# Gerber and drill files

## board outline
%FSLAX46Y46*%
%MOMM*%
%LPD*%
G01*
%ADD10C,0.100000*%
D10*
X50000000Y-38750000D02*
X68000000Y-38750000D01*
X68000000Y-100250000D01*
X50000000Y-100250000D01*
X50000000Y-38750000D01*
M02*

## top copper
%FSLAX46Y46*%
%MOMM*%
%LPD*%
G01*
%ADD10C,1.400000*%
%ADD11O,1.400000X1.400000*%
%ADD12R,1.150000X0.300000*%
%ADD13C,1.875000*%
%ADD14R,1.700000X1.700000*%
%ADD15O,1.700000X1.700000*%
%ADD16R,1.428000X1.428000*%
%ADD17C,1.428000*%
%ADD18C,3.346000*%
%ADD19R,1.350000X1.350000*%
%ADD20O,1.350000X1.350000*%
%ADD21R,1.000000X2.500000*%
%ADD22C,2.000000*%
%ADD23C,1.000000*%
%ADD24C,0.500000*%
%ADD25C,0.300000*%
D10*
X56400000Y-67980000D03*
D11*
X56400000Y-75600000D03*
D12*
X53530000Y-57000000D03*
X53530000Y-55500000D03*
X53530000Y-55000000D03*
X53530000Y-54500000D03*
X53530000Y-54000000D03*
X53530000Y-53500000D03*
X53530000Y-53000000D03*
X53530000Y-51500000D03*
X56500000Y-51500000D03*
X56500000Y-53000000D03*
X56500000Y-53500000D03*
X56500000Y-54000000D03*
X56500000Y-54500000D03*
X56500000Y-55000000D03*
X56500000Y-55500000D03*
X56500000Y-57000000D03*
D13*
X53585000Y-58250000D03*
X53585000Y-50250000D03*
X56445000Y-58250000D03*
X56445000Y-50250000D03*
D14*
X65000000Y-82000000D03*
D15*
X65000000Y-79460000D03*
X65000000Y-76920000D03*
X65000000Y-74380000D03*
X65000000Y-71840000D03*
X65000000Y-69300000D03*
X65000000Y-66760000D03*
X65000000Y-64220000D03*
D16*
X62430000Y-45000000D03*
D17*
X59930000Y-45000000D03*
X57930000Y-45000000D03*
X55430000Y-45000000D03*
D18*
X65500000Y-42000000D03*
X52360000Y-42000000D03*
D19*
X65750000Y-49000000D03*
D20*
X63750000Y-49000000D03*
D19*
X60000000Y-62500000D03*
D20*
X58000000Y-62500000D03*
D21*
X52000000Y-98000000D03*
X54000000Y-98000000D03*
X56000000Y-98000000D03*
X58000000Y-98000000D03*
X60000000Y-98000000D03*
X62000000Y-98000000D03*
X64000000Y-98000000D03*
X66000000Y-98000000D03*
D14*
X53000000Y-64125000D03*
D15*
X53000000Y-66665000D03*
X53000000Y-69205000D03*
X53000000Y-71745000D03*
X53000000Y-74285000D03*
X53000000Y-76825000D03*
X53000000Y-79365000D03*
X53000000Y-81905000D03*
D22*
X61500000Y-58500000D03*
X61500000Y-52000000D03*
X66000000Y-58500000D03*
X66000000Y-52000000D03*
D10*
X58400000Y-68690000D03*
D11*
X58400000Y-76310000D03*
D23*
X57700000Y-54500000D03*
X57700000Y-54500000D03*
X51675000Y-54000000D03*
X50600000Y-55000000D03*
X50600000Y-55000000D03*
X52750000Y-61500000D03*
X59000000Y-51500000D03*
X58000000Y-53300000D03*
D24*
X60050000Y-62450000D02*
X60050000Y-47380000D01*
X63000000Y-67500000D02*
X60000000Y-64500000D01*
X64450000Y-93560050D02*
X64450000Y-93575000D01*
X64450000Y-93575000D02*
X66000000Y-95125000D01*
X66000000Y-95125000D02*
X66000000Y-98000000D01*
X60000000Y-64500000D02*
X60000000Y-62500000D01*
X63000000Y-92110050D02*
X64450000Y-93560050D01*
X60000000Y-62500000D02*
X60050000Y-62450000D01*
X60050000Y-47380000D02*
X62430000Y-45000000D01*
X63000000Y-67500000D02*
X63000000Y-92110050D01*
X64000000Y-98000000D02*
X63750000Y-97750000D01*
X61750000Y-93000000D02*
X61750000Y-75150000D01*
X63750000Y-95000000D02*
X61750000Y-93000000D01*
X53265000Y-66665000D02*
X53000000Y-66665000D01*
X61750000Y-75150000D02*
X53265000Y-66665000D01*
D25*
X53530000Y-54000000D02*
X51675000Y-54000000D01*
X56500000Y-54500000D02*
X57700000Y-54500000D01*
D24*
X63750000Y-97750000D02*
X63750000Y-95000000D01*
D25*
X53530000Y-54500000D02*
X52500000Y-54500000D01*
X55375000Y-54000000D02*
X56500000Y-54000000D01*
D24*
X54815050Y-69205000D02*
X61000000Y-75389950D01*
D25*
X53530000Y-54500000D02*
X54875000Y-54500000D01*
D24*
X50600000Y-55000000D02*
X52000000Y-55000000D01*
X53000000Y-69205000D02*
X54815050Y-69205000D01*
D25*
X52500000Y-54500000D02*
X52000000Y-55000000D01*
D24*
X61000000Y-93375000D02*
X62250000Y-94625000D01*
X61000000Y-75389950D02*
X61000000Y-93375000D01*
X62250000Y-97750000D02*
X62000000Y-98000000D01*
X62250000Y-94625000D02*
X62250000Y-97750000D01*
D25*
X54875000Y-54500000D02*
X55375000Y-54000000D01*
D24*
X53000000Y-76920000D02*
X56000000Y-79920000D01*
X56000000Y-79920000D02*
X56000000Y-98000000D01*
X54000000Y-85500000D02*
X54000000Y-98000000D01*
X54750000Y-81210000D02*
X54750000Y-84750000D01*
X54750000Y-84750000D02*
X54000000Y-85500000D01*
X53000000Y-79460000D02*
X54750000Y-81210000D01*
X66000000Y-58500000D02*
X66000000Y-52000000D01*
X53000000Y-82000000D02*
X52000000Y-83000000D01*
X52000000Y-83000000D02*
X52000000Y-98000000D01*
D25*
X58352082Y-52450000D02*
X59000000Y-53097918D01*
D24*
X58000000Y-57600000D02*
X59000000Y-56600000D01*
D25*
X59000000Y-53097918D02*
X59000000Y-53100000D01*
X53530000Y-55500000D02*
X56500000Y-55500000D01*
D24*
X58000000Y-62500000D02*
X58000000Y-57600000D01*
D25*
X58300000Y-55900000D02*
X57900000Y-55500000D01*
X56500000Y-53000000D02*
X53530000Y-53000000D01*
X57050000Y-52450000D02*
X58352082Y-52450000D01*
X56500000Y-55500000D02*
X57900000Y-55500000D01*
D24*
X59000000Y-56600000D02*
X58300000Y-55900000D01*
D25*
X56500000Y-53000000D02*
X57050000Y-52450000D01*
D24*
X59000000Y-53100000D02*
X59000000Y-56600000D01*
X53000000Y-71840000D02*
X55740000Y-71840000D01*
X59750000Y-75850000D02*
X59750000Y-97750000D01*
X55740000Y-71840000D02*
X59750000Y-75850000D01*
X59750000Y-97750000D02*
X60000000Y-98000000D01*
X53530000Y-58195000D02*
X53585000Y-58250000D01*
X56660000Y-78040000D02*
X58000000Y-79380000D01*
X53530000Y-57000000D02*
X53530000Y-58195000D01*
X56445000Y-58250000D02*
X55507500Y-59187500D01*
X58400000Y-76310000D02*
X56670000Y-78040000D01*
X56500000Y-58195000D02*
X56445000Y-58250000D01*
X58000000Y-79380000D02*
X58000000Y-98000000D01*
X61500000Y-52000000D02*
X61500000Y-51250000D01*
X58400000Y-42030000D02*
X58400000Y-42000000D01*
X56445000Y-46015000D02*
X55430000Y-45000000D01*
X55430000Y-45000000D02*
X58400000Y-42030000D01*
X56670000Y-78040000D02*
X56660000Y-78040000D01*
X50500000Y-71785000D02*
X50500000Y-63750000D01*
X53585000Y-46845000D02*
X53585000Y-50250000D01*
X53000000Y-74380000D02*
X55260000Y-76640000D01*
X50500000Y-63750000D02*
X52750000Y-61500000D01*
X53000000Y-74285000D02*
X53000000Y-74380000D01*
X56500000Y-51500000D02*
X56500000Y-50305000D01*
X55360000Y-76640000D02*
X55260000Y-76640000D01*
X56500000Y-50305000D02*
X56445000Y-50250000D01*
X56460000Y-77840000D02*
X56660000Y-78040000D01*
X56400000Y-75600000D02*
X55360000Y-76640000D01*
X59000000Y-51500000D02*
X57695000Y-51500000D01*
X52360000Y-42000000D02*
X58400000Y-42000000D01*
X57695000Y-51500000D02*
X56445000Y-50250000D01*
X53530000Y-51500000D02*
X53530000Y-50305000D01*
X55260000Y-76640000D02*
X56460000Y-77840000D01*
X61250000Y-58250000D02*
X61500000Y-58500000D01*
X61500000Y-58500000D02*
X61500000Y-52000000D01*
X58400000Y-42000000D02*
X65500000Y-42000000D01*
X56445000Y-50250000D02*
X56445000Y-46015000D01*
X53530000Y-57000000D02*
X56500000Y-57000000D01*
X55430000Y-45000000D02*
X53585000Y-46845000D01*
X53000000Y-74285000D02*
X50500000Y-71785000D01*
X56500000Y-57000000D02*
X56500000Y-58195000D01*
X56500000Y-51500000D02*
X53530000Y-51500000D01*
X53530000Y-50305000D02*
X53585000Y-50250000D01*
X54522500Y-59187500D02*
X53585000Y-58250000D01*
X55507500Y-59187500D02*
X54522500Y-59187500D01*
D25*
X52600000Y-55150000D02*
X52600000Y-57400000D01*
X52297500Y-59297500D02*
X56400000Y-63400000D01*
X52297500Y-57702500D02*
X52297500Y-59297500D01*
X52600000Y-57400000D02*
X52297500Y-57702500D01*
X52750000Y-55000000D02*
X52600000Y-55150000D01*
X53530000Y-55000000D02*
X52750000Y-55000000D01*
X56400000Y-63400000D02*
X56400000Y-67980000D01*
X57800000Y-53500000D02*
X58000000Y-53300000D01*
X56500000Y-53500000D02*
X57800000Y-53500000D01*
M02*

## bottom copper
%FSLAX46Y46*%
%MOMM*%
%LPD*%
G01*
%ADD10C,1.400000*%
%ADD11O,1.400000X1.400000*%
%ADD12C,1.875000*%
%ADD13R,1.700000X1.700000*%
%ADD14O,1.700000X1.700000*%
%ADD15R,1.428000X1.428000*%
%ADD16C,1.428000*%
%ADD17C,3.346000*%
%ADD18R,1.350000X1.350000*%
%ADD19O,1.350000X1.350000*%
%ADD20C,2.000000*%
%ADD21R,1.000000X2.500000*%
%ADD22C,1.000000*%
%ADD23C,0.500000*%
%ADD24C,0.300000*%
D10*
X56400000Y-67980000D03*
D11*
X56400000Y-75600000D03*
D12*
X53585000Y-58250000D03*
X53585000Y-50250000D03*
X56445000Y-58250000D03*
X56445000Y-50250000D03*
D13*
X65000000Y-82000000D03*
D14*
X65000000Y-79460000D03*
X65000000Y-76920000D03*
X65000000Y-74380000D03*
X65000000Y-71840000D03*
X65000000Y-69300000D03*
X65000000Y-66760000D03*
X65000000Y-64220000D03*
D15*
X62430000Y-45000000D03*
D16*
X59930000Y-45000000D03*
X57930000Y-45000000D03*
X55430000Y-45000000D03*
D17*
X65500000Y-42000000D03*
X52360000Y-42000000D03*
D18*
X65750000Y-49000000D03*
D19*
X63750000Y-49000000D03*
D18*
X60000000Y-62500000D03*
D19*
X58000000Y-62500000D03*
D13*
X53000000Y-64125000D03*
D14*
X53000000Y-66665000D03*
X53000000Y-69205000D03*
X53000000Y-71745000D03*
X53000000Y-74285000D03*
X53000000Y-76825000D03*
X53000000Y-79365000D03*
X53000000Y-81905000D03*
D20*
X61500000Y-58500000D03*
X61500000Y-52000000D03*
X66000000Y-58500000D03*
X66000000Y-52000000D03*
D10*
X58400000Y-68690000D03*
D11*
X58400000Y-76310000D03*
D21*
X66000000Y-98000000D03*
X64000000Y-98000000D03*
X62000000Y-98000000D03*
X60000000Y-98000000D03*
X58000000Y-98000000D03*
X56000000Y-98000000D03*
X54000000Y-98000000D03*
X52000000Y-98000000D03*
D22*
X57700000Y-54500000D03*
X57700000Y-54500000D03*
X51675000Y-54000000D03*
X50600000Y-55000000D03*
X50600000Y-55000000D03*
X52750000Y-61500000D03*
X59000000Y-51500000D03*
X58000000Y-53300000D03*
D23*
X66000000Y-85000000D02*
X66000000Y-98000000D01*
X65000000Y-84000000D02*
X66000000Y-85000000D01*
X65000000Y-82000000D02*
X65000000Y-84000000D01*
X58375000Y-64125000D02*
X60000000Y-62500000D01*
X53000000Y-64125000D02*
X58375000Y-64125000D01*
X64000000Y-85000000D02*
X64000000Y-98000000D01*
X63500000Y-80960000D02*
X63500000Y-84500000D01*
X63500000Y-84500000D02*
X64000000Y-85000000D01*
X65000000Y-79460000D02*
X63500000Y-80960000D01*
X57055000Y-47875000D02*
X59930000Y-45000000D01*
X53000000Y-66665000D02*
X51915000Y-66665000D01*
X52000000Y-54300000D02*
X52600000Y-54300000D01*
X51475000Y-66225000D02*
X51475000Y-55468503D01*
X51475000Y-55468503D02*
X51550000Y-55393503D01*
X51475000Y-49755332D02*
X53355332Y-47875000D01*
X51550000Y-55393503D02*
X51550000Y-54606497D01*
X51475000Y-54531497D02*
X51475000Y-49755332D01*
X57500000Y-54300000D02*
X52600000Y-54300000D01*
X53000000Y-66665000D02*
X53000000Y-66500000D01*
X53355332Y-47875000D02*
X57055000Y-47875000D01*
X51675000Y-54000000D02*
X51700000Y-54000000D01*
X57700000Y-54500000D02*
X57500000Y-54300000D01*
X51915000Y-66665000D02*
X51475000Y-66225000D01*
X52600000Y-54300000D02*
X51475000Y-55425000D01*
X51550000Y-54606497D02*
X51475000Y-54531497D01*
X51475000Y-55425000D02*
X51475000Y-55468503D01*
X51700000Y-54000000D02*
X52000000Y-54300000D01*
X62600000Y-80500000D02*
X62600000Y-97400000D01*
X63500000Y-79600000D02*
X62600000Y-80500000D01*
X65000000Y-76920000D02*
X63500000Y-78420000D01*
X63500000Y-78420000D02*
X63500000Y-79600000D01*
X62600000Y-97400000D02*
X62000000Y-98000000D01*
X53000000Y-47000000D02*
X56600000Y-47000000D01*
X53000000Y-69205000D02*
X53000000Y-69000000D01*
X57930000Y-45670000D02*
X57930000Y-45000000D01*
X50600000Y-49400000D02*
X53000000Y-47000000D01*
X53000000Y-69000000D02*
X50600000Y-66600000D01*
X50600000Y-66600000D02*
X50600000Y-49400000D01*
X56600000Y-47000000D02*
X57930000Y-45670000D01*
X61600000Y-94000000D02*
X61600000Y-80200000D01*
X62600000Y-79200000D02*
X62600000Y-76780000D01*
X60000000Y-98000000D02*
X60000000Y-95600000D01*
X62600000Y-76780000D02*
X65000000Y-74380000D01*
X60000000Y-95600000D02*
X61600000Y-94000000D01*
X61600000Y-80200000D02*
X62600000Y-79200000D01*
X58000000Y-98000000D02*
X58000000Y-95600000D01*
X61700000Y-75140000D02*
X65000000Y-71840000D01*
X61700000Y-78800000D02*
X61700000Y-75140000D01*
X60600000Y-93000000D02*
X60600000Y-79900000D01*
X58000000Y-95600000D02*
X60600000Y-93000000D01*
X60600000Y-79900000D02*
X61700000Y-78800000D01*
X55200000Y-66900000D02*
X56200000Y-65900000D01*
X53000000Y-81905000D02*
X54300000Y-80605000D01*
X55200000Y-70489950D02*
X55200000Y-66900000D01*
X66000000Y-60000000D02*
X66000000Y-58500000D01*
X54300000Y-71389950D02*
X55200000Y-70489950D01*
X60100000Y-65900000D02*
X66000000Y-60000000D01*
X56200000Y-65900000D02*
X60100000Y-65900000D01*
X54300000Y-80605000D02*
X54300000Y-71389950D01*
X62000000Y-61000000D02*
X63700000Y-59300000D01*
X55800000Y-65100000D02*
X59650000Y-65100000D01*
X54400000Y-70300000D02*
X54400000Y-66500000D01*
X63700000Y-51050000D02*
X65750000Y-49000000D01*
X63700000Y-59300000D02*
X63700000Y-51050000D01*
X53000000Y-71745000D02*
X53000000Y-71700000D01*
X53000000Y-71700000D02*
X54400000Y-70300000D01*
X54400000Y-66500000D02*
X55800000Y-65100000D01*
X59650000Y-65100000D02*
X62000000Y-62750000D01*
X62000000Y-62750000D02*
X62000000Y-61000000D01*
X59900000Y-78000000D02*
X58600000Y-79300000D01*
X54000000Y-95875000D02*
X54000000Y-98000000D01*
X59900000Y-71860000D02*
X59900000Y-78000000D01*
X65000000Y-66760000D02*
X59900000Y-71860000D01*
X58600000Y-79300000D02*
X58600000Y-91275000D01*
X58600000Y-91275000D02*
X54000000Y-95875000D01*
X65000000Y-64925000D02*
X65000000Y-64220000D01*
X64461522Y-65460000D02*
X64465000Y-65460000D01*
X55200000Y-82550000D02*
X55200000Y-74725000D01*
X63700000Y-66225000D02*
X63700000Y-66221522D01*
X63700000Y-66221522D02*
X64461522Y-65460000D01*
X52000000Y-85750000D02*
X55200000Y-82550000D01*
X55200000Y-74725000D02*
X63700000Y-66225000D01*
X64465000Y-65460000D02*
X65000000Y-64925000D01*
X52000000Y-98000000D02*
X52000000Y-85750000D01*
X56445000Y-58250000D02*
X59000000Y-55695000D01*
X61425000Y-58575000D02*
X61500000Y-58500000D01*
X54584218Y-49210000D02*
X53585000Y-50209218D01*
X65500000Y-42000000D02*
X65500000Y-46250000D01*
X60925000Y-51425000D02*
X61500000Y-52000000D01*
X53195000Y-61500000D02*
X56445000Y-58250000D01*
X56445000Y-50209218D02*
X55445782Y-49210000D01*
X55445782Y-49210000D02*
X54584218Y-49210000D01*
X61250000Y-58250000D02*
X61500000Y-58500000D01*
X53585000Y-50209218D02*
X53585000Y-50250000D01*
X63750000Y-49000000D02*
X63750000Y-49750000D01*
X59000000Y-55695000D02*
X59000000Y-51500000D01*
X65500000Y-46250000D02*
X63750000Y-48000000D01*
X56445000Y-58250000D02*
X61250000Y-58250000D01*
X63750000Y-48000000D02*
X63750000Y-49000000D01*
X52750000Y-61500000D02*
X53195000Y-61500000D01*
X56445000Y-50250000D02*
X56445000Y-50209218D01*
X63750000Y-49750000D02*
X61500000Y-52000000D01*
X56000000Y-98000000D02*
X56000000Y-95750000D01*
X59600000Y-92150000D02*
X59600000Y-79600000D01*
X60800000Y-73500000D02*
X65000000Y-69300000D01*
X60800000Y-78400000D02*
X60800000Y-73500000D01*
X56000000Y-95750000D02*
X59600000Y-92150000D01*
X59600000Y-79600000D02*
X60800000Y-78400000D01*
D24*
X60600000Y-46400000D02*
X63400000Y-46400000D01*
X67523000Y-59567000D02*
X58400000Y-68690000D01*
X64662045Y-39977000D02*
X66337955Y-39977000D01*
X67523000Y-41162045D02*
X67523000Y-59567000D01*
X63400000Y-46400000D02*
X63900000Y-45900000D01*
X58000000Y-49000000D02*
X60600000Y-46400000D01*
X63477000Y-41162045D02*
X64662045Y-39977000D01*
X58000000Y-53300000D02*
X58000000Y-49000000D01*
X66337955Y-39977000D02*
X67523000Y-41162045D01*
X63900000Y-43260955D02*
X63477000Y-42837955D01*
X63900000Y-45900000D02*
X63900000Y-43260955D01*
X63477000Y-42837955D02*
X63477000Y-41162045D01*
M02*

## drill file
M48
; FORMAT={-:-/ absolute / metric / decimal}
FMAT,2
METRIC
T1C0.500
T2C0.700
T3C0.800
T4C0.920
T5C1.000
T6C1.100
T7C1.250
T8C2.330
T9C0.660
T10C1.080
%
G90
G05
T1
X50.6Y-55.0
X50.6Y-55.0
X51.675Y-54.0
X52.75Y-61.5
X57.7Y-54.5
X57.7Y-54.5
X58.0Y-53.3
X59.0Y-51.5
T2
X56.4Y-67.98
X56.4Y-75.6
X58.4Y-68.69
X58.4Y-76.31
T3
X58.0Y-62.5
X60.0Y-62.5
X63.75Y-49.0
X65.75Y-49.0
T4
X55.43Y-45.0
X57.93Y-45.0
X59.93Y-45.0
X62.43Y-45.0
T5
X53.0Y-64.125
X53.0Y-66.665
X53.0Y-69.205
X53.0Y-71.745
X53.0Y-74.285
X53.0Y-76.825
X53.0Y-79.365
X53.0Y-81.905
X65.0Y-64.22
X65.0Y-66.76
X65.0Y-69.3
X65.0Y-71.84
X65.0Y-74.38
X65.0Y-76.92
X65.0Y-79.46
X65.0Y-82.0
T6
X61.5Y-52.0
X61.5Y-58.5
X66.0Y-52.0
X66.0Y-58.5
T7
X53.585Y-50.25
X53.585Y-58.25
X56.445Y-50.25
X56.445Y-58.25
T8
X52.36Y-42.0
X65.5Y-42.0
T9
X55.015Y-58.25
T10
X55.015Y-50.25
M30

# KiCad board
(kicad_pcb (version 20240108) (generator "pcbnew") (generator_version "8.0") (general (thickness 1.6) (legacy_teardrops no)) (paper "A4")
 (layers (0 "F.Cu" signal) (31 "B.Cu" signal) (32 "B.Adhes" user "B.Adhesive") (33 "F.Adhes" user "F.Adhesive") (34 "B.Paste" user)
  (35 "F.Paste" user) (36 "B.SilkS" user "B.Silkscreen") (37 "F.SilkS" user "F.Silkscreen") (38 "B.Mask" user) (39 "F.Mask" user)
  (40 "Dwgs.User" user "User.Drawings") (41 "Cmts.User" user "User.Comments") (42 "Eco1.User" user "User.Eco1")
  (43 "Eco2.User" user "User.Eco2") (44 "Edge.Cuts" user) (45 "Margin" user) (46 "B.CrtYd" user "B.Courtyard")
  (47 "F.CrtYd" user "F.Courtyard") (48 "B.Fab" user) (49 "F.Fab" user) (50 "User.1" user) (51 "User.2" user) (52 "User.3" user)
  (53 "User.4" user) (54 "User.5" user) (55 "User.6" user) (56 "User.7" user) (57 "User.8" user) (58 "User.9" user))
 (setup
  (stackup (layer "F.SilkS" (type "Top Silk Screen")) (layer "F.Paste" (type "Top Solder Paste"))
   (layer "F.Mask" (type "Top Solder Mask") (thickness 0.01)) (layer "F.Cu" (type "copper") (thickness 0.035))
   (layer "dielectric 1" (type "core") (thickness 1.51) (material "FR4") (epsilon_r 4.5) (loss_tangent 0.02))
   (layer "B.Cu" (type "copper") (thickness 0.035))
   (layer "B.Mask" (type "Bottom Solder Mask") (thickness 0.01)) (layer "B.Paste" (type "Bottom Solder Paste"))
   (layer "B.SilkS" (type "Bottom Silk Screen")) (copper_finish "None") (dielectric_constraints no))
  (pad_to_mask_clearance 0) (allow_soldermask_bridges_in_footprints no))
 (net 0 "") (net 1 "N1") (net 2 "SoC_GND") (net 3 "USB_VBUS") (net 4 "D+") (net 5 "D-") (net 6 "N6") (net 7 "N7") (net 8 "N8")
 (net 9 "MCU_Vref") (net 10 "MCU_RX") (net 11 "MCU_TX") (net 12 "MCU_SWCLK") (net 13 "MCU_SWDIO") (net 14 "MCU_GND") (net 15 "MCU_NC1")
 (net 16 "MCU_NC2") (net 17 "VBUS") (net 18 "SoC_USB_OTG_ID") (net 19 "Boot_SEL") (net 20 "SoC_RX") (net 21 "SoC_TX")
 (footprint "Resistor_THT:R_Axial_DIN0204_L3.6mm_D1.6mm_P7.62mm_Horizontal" (layer "F.Cu") (at 56.4 67.98 -90)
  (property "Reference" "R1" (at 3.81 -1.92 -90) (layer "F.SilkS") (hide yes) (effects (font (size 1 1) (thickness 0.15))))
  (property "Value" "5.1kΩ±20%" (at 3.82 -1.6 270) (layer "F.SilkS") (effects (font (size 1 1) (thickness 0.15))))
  (pad "1" thru_hole circle (at 0 0 270) (size 1.4 1.4) (drill 0.7) (layers "*.Cu" "*.Mask") (remove_unused_layers no) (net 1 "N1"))
  (pad "2" thru_hole oval (at 7.62 0 270) (size 1.4 1.4) (drill 0.7) (layers "*.Cu" "*.Mask") (remove_unused_layers no) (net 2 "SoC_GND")))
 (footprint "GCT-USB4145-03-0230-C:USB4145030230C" (layer "F.Cu") (at 55.015 54.25 90)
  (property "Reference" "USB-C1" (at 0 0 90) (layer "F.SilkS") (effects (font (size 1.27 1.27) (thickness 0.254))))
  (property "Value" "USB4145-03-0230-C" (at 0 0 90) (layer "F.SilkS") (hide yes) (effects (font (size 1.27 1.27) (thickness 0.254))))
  (pad "" np_thru_hole circle (at -4 0 90) (size 0.66 0.66) (drill 0.66) (layers "*.Cu" "*.Mask"))
  (pad "" np_thru_hole circle (at 4 0 90) (size 1.08 1.08) (drill 1.08) (layers "*.Cu" "*.Mask"))
  (pad "A1" smd rect (at -2.75 -1.485 90) (size 0.3 1.15) (layers "F.Cu" "F.Mask") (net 2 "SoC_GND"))
  (pad "A4" smd rect (at -1.25 -1.485 90) (size 0.3 1.15) (layers "F.Cu" "F.Mask") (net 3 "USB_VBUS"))
  (pad "A5" smd rect (at -0.75 -1.485 90) (size 0.3 1.15) (layers "F.Cu" "F.Mask") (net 1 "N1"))
  (pad "A6" smd rect (at -0.25 -1.485 90) (size 0.3 1.15) (layers "F.Cu" "F.Mask") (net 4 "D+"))
  (pad "A7" smd rect (at 0.25 -1.485 90) (size 0.3 1.15) (layers "F.Cu" "F.Mask") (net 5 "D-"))
  (pad "A8" smd rect (at 0.75 -1.485 90) (size 0.3 1.15) (layers "F.Cu" "F.Mask") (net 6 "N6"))
  (pad "A9" smd rect (at 1.25 -1.485 90) (size 0.3 1.15) (layers "F.Cu" "F.Mask") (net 3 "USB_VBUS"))
  (pad "A12" smd rect (at 2.75 -1.485 90) (size 0.3 1.15) (layers "F.Cu" "F.Mask") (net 2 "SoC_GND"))
  (pad "B1" smd rect (at 2.75 1.485 90) (size 0.3 1.15) (layers "F.Cu" "F.Mask") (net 2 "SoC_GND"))
  (pad "B4" smd rect (at 1.25 1.485 90) (size 0.3 1.15) (layers "F.Cu" "F.Mask") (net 3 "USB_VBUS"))
  (pad "B5" smd rect (at 0.75 1.485 90) (size 0.3 1.15) (layers "F.Cu" "F.Mask") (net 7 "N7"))
  (pad "B6" smd rect (at 0.25 1.485 90) (size 0.3 1.15) (layers "F.Cu" "F.Mask") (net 4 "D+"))
  (pad "B7" smd rect (at -0.25 1.485 90) (size 0.3 1.15) (layers "F.Cu" "F.Mask") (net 5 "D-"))
  (pad "B8" smd rect (at -0.75 1.485 90) (size 0.3 1.15) (layers "F.Cu" "F.Mask") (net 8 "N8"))
  (pad "B9" smd rect (at -1.25 1.485 90) (size 0.3 1.15) (layers "F.Cu" "F.Mask") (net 3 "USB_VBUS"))
  (pad "B12" smd rect (at -2.75 1.485 90) (size 0.3 1.15) (layers "F.Cu" "F.Mask") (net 2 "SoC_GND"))
  (pad "MH1" thru_hole circle (at -4 -1.43 90) (size 1.875 1.875) (drill 1.25) (layers "*.Cu" "*.Mask") (remove_unused_layers no)
   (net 2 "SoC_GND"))
  (pad "MH2" thru_hole circle (at 4 -1.43 90) (size 1.875 1.875) (drill 1.25) (layers "*.Cu" "*.Mask") (remove_unused_layers no)
   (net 2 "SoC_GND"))
  (pad "MH3" thru_hole circle (at -4 1.43 90) (size 1.875 1.875) (drill 1.25) (layers "*.Cu" "*.Mask") (remove_unused_layers no)
   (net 2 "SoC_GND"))
  (pad "MH4" thru_hole circle (at 4 1.43 90) (size 1.875 1.875) (drill 1.25) (layers "*.Cu" "*.Mask") (remove_unused_layers no)
   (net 2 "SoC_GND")))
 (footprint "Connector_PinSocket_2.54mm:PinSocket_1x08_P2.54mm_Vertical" (layer "F.Cu") (at 65 82 180)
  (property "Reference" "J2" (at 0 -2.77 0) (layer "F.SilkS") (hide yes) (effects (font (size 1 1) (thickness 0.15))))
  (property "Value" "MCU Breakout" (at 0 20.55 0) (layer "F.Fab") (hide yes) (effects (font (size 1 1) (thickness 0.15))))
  (pad "1" thru_hole rect (at 0 0 180) (size 1.7 1.7) (drill 1) (layers "*.Cu" "*.Mask") (remove_unused_layers yes) (keep_end_layers yes)
   (zone_layer_connections) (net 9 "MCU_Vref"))
  (pad "2" thru_hole oval (at 0 2.54 180) (size 1.7 1.7) (drill 1) (layers "*.Cu" "*.Mask") (remove_unused_layers yes) (keep_end_layers yes)
   (zone_layer_connections) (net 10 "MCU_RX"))
  (pad "3" thru_hole oval (at 0 5.08 180) (size 1.7 1.7) (drill 1) (layers "*.Cu" "*.Mask") (remove_unused_layers yes) (keep_end_layers yes)
   (zone_layer_connections) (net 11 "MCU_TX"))
  (pad "4" thru_hole oval (at 0 7.62 180) (size 1.7 1.7) (drill 1) (layers "*.Cu" "*.Mask") (remove_unused_layers yes) (keep_end_layers yes)
   (zone_layer_connections) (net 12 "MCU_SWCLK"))
  (pad "5" thru_hole oval (at 0 10.16 180) (size 1.7 1.7) (drill 1) (layers "*.Cu" "*.Mask") (remove_unused_layers yes)
   (keep_end_layers yes) (zone_layer_connections) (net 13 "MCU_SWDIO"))
  (pad "6" thru_hole oval (at 0 12.7 180) (size 1.7 1.7) (drill 1) (layers "*.Cu" "*.Mask") (remove_unused_layers yes) (keep_end_layers yes)
   (zone_layer_connections) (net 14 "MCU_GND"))
  (pad "7" thru_hole oval (at 0 15.24 180) (size 1.7 1.7) (drill 1) (layers "*.Cu" "*.Mask") (remove_unused_layers yes)
   (keep_end_layers yes) (zone_layer_connections) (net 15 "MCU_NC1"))
  (pad "8" thru_hole oval (at 0 17.78 180) (size 1.7 1.7) (drill 1) (layers "*.Cu" "*.Mask") (remove_unused_layers yes)
   (keep_end_layers yes) (zone_layer_connections) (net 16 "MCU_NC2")))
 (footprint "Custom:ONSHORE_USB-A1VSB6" (layer "F.Cu") (at 58.93 42 180)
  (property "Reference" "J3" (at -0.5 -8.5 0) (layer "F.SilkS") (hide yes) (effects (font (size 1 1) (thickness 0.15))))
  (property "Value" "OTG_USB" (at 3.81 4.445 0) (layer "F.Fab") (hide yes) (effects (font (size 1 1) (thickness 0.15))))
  (pad "1" thru_hole rect (at -3.5 -3 180) (size 1.428 1.428) (drill 0.92) (layers "*.Cu" "*.Mask") (remove_unused_layers yes)
   (keep_end_layers yes) (zone_layer_connections) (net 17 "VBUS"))
  (pad "2" thru_hole circle (at -1 -3 180) (size 1.428 1.428) (drill 0.92) (layers "*.Cu" "*.Mask") (remove_unused_layers yes)
   (keep_end_layers yes) (zone_layer_connections) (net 5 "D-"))
  (pad "3" thru_hole circle (at 1 -3 180) (size 1.428 1.428) (drill 0.92) (layers "*.Cu" "*.Mask") (remove_unused_layers yes)
   (keep_end_layers yes) (zone_layer_connections) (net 4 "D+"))
  (pad "4" thru_hole circle (at 3.5 -3 180) (size 1.428 1.428) (drill 0.92) (layers "*.Cu" "*.Mask") (remove_unused_layers yes)
   (keep_end_layers yes) (zone_layer_connections) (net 2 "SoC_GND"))
  (pad "S1" thru_hole circle (at -6.57 0 180) (size 3.346 3.346) (drill 2.33) (layers "*.Cu" "*.Mask") (remove_unused_layers yes)
   (keep_end_layers yes) (zone_layer_connections))
  (pad "S2" thru_hole circle (at 6.57 0 180) (size 3.346 3.346) (drill 2.33) (layers "*.Cu" "*.Mask") (remove_unused_layers yes)
   (keep_end_layers yes) (zone_layer_connections)))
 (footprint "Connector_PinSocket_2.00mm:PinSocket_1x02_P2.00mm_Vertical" (layer "F.Cu") (at 65.75 49 -90)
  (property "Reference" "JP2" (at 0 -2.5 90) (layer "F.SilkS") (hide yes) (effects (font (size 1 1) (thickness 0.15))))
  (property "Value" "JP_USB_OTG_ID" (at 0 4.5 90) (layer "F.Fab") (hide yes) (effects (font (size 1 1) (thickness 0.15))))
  (pad "1" thru_hole rect (at 0 0 270) (size 1.35 1.35) (drill 0.8) (layers "*.Cu" "*.Mask") (remove_unused_layers yes)
   (keep_end_layers yes) (zone_layer_connections) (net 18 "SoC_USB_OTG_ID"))
  (pad "2" thru_hole oval (at 0 2 270) (size 1.35 1.35) (drill 0.8) (layers "*.Cu" "*.Mask") (remove_unused_layers yes)
   (keep_end_layers yes) (zone_layer_connections) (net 2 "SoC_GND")))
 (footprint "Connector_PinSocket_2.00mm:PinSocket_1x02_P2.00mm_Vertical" (layer "F.Cu") (at 60 62.5 -90)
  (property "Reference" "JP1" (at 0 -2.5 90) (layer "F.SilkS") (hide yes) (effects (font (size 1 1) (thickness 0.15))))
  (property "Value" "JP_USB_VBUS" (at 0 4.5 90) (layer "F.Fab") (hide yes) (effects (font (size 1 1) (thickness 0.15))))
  (pad "1" thru_hole rect (at 0 0 270) (size 1.35 1.35) (drill 0.8) (layers "*.Cu" "*.Mask") (remove_unused_layers yes)
   (keep_end_layers yes) (zone_layer_connections) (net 17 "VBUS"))
  (pad "2" thru_hole oval (at 0 2 270) (size 1.35 1.35) (drill 0.8) (layers "*.Cu" "*.Mask") (remove_unused_layers yes)
   (keep_end_layers yes) (zone_layer_connections) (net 3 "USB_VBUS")))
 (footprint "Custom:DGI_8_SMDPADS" (layer "F.Cu") (at 59 98)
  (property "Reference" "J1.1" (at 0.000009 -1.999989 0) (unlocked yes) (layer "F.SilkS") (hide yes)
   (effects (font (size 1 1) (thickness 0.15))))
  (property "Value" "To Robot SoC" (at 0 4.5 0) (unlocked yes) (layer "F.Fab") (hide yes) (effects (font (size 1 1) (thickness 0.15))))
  (pad "1" smd rect (at -7 0) (size 1 2.5) (layers "F.Cu" "F.Paste" "F.Mask") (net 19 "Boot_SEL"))
  (pad "2" smd rect (at -5 0) (size 1 2.5) (layers "F.Cu" "F.Paste" "F.Mask") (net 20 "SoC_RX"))
  (pad "3" smd rect (at -3 0) (size 1 2.5) (layers "F.Cu" "F.Paste" "F.Mask") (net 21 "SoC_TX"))
  (pad "4" smd rect (at -1 0) (size 1 2.5) (layers "F.Cu" "F.Paste" "F.Mask") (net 2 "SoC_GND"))
  (pad "5" smd rect (at 1 0) (size 1 2.5) (layers "F.Cu" "F.Paste" "F.Mask") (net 18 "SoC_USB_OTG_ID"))
  (pad "6" smd rect (at 3 0) (size 1 2.5) (layers "F.Cu" "F.Paste" "F.Mask") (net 4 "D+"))
  (pad "7" smd rect (at 5 0) (size 1 2.5) (layers "F.Cu" "F.Paste" "F.Mask") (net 5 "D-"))
  (pad "8" smd rect (at 7 0) (size 1 2.5) (layers "F.Cu" "F.Paste" "F.Mask") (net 17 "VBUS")))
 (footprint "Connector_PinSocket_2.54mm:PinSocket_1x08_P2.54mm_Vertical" (layer "F.Cu") (at 53 64.125)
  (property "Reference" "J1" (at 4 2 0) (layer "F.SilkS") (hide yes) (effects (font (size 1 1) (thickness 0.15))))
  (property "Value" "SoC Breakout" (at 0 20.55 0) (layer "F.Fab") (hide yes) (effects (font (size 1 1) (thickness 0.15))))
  (pad "1" thru_hole rect (at 0 0) (size 1.7 1.7) (drill 1) (layers "*.Cu" "*.Mask") (remove_unused_layers yes) (keep_end_layers yes)
   (zone_layer_connections) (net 17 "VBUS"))
  (pad "2" thru_hole oval (at 0 2.54) (size 1.7 1.7) (drill 1) (layers "*.Cu" "*.Mask") (remove_unused_layers yes) (keep_end_layers yes)
   (zone_layer_connections) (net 5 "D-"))
  (pad "3" thru_hole oval (at 0 5.08) (size 1.7 1.7) (drill 1) (layers "*.Cu" "*.Mask") (remove_unused_layers yes) (keep_end_layers yes)
   (zone_layer_connections) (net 4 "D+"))
  (pad "4" thru_hole oval (at 0 7.62) (size 1.7 1.7) (drill 1) (layers "*.Cu" "*.Mask") (remove_unused_layers yes) (keep_end_layers yes)
   (zone_layer_connections) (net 18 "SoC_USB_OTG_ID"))
  (pad "5" thru_hole oval (at 0 10.16) (size 1.7 1.7) (drill 1) (layers "*.Cu" "*.Mask") (remove_unused_layers yes) (keep_end_layers yes)
   (zone_layer_connections) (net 2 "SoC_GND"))
  (pad "6" thru_hole oval (at 0 12.7) (size 1.7 1.7) (drill 1) (layers "*.Cu" "*.Mask") (remove_unused_layers yes) (keep_end_layers yes)
   (zone_layer_connections) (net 21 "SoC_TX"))
  (pad "7" thru_hole oval (at 0 15.24) (size 1.7 1.7) (drill 1) (layers "*.Cu" "*.Mask") (remove_unused_layers yes) (keep_end_layers yes)
   (zone_layer_connections) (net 20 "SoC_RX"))
  (pad "8" thru_hole oval (at 0 17.78) (size 1.7 1.7) (drill 1) (layers "*.Cu" "*.Mask") (remove_unused_layers yes) (keep_end_layers yes)
   (zone_layer_connections) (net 19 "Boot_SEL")))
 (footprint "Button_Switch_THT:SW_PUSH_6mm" (layer "F.Cu") (at 61.5 58.5 90)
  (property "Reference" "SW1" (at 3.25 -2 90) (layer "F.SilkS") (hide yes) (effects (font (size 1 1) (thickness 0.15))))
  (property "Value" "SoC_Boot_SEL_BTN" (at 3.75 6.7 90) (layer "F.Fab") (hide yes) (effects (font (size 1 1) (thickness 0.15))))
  (pad "1" thru_hole circle (at 0 0 180) (size 2 2) (drill 1.1) (layers "*.Cu" "*.Mask") (remove_unused_layers yes) (keep_end_layers yes)
   (zone_layer_connections) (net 2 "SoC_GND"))
  (pad "1" thru_hole circle (at 6.5 0 180) (size 2 2) (drill 1.1) (layers "*.Cu" "*.Mask") (remove_unused_layers yes) (keep_end_layers yes)
   (zone_layer_connections) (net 2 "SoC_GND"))
  (pad "2" thru_hole circle (at 0 4.5 180) (size 2 2) (drill 1.1) (layers "*.Cu" "*.Mask") (remove_unused_layers yes) (keep_end_layers yes)
   (zone_layer_connections) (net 19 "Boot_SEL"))
  (pad "2" thru_hole circle (at 6.5 4.5 180) (size 2 2) (drill 1.1) (layers "*.Cu" "*.Mask") (remove_unused_layers yes)
   (keep_end_layers yes) (zone_layer_connections) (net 19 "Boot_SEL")))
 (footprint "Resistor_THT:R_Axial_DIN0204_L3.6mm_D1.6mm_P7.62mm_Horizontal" (layer "F.Cu") (at 58.4 68.69 -90)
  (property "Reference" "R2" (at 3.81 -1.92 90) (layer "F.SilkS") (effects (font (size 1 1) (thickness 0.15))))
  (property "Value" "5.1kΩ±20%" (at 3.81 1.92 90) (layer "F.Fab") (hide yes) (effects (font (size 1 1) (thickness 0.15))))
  (pad "1" thru_hole circle (at 0 0 270) (size 1.4 1.4) (drill 0.7) (layers "*.Cu" "*.Mask") (remove_unused_layers no) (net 7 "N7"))
  (pad "2" thru_hole oval (at 7.62 0 270) (size 1.4 1.4) (drill 0.7) (layers "*.Cu" "*.Mask") (remove_unused_layers no) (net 2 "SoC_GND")))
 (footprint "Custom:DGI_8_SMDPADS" (layer "B.Cu") (at 59 98 180)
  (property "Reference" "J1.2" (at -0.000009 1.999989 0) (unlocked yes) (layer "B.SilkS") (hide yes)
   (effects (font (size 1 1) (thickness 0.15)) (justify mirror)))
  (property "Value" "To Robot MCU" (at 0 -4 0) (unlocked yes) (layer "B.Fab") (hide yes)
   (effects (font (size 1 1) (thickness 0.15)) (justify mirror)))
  (pad "1" smd rect (at -7 0 180) (size 1 2.5) (layers "B.Cu" "B.Paste" "B.Mask") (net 9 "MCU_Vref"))
  (pad "2" smd rect (at -5 0 180) (size 1 2.5) (layers "B.Cu" "B.Paste" "B.Mask") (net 10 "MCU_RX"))
  (pad "3" smd rect (at -3 0 180) (size 1 2.5) (layers "B.Cu" "B.Paste" "B.Mask") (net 11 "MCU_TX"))
  (pad "4" smd rect (at -1 0 180) (size 1 2.5) (layers "B.Cu" "B.Paste" "B.Mask") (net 12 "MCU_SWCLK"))
  (pad "5" smd rect (at 1 0 180) (size 1 2.5) (layers "B.Cu" "B.Paste" "B.Mask") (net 13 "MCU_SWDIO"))
  (pad "6" smd rect (at 3 0 180) (size 1 2.5) (layers "B.Cu" "B.Paste" "B.Mask") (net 14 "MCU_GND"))
  (pad "7" smd rect (at 5 0 180) (size 1 2.5) (layers "B.Cu" "B.Paste" "B.Mask") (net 15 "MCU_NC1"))
  (pad "8" smd rect (at 7 0 180) (size 1 2.5) (layers "B.Cu" "B.Paste" "B.Mask") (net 16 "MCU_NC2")))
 (gr_rect (start 50 38.75) (end 68 100.25) (stroke (width 0.1) (type solid)) (fill none) (layer "Edge.Cuts"))
 (segment (start 66 85) (end 66 98) (width 0.5) (layer "B.Cu") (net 9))
 (segment (start 65 84) (end 66 85) (width 0.5) (layer "B.Cu") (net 9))
 (segment (start 65 82) (end 65 84) (width 0.5) (layer "B.Cu") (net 9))
 (segment (start 60.05 62.45) (end 60.05 47.38) (width 0.5) (layer "F.Cu") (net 17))
 (segment (start 63 67.5) (end 60 64.5) (width 0.5) (layer "F.Cu") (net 17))
 (segment (start 64.45 93.56005) (end 64.45 93.575) (width 0.5) (layer "F.Cu") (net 17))
 (segment (start 64.45 93.575) (end 66 95.125) (width 0.5) (layer "F.Cu") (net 17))
 (segment (start 66 95.125) (end 66 98) (width 0.5) (layer "F.Cu") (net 17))
 (segment (start 60 64.5) (end 60 62.5) (width 0.5) (layer "F.Cu") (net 17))
 (segment (start 63 92.11005) (end 64.45 93.56005) (width 0.5) (layer "F.Cu") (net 17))
 (segment (start 60 62.5) (end 60.05 62.45) (width 0.5) (layer "F.Cu") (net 17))
 (segment (start 60.05 47.38) (end 62.43 45) (width 0.5) (layer "F.Cu") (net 17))
 (segment (start 63 67.5) (end 63 92.11005) (width 0.5) (layer "F.Cu") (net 17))
 (segment (start 58.375 64.125) (end 60 62.5) (width 0.5) (layer "B.Cu") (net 17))
 (segment (start 53 64.125) (end 58.375 64.125) (width 0.5) (layer "B.Cu") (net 17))
 (segment (start 64 85) (end 64 98) (width 0.5) (layer "B.Cu") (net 10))
 (segment (start 63.5 80.96) (end 63.5 84.5) (width 0.5) (layer "B.Cu") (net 10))
 (segment (start 63.5 84.5) (end 64 85) (width 0.5) (layer "B.Cu") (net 10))
 (segment (start 65 79.46) (end 63.5 80.96) (width 0.5) (layer "B.Cu") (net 10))
 (segment (start 64 98) (end 63.75 97.75) (width 0.5) (layer "F.Cu") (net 5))
 (segment (start 61.75 93) (end 61.75 75.15) (width 0.5) (layer "F.Cu") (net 5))
 (segment (start 63.75 95) (end 61.75 93) (width 0.5) (layer "F.Cu") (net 5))
 (segment (start 53.265 66.665) (end 53 66.665) (width 0.5) (layer "F.Cu") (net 5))
 (segment (start 61.75 75.15) (end 53.265 66.665) (width 0.5) (layer "F.Cu") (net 5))
 (segment (start 53.53 54) (end 51.675 54) (width 0.3) (layer "F.Cu") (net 5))
 (segment (start 56.5 54.5) (end 57.7 54.5) (width 0.3) (layer "F.Cu") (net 5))
 (segment (start 63.75 97.75) (end 63.75 95) (width 0.5) (layer "F.Cu") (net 5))
 (via (at 57.7 54.5) (size 1) (drill 0.5) (layers "F.Cu" "B.Cu") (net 5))
 (via (at 57.7 54.5) (size 1) (drill 0.5) (layers "F.Cu" "B.Cu") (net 5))
 (via (at 51.675 54) (size 1) (drill 0.5) (layers "F.Cu" "B.Cu") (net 5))
 (segment (start 57.055 47.875) (end 59.93 45) (width 0.5) (layer "B.Cu") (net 5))
 (segment (start 53 66.665) (end 51.915 66.665) (width 0.5) (layer "B.Cu") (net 5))
 (segment (start 52 54.3) (end 52.6 54.3) (width 0.5) (layer "B.Cu") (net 5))
 (segment (start 51.475 66.225) (end 51.475 55.468503) (width 0.5) (layer "B.Cu") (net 5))
 (segment (start 51.475 55.468503) (end 51.55 55.393503) (width 0.5) (layer "B.Cu") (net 5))
 (segment (start 51.475 49.755332) (end 53.355332 47.875) (width 0.5) (layer "B.Cu") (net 5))
 (segment (start 51.55 55.393503) (end 51.55 54.606497) (width 0.5) (layer "B.Cu") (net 5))
 (segment (start 51.475 54.531497) (end 51.475 49.755332) (width 0.5) (layer "B.Cu") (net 5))
 (segment (start 57.5 54.3) (end 52.6 54.3) (width 0.5) (layer "B.Cu") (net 5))
 (segment (start 53 66.665) (end 53 66.5) (width 0.5) (layer "B.Cu") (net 5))
 (segment (start 53.355332 47.875) (end 57.055 47.875) (width 0.5) (layer "B.Cu") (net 5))
 (segment (start 51.675 54) (end 51.7 54) (width 0.5) (layer "B.Cu") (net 5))
 (segment (start 57.7 54.5) (end 57.5 54.3) (width 0.5) (layer "B.Cu") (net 5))
 (segment (start 51.915 66.665) (end 51.475 66.225) (width 0.5) (layer "B.Cu") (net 5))
 (segment (start 52.6 54.3) (end 51.475 55.425) (width 0.5) (layer "B.Cu") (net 5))
 (segment (start 51.55 54.606497) (end 51.475 54.531497) (width 0.5) (layer "B.Cu") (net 5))
 (segment (start 51.475 55.425) (end 51.475 55.468503) (width 0.5) (layer "B.Cu") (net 5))
 (segment (start 51.7 54) (end 52 54.3) (width 0.5) (layer "B.Cu") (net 5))
 (segment (start 62.6 80.5) (end 62.6 97.4) (width 0.5) (layer "B.Cu") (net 11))
 (segment (start 63.5 79.6) (end 62.6 80.5) (width 0.5) (layer "B.Cu") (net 11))
 (segment (start 65 76.92) (end 63.5 78.42) (width 0.5) (layer "B.Cu") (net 11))
 (segment (start 63.5 78.42) (end 63.5 79.6) (width 0.5) (layer "B.Cu") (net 11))
 (segment (start 62.6 97.4) (end 62 98) (width 0.5) (layer "B.Cu") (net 11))
 (segment (start 53.53 54.5) (end 52.5 54.5) (width 0.3) (layer "F.Cu") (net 4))
 (segment (start 55.375 54) (end 56.5 54) (width 0.3) (layer "F.Cu") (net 4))
 (segment (start 54.81505 69.205) (end 61 75.38995) (width 0.5) (layer "F.Cu") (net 4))
 (segment (start 53.53 54.5) (end 54.875 54.5) (width 0.3) (layer "F.Cu") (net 4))
 (segment (start 50.6 55) (end 52 55) (width 0.5) (layer "F.Cu") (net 4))
 (segment (start 53 69.205) (end 54.81505 69.205) (width 0.5) (layer "F.Cu") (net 4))
 (segment (start 52.5 54.5) (end 52 55) (width 0.3) (layer "F.Cu") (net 4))
 (segment (start 61 93.375) (end 62.25 94.625) (width 0.5) (layer "F.Cu") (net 4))
 (segment (start 61 75.38995) (end 61 93.375) (width 0.5) (layer "F.Cu") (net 4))
 (segment (start 62.25 97.75) (end 62 98) (width 0.5) (layer "F.Cu") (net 4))
 (segment (start 62.25 94.625) (end 62.25 97.75) (width 0.5) (layer "F.Cu") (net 4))
 (segment (start 54.875 54.5) (end 55.375 54) (width 0.3) (layer "F.Cu") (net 4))
 (via (at 50.6 55) (size 1) (drill 0.5) (layers "F.Cu" "B.Cu") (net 4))
 (via (at 50.6 55) (size 1) (drill 0.5) (layers "F.Cu" "B.Cu") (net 4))
 (segment (start 53 47) (end 56.6 47) (width 0.5) (layer "B.Cu") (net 4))
 (segment (start 53 69.205) (end 53 69) (width 0.5) (layer "B.Cu") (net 4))
 (segment (start 57.93 45.67) (end 57.93 45) (width 0.5) (layer "B.Cu") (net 4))
 (segment (start 50.6 49.4) (end 53 47) (width 0.5) (layer "B.Cu") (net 4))
 (segment (start 53 69) (end 50.6 66.6) (width 0.5) (layer "B.Cu") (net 4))
 (segment (start 50.6 66.6) (end 50.6 49.4) (width 0.5) (layer "B.Cu") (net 4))
 (segment (start 56.6 47) (end 57.93 45.67) (width 0.5) (layer "B.Cu") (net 4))
 (segment (start 61.6 94) (end 61.6 80.2) (width 0.5) (layer "B.Cu") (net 12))
 (segment (start 62.6 79.2) (end 62.6 76.78) (width 0.5) (layer "B.Cu") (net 12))
 (segment (start 60 98) (end 60 95.6) (width 0.5) (layer "B.Cu") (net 12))
 (segment (start 62.6 76.78) (end 65 74.38) (width 0.5) (layer "B.Cu") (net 12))
 (segment (start 60 95.6) (end 61.6 94) (width 0.5) (layer "B.Cu") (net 12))
 (segment (start 61.6 80.2) (end 62.6 79.2) (width 0.5) (layer "B.Cu") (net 12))
 (segment (start 58 98) (end 58 95.6) (width 0.5) (layer "B.Cu") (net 13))
 (segment (start 61.7 75.14) (end 65 71.84) (width 0.5) (layer "B.Cu") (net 13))
 (segment (start 61.7 78.8) (end 61.7 75.14) (width 0.5) (layer "B.Cu") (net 13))
 (segment (start 60.6 93) (end 60.6 79.9) (width 0.5) (layer "B.Cu") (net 13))
 (segment (start 58 95.6) (end 60.6 93) (width 0.5) (layer "B.Cu") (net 13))
 (segment (start 60.6 79.9) (end 61.7 78.8) (width 0.5) (layer "B.Cu") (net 13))
 (segment (start 53 76.92) (end 56 79.92) (width 0.5) (layer "F.Cu") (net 21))
 (segment (start 56 79.92) (end 56 98) (width 0.5) (layer "F.Cu") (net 21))
 (segment (start 54 85.5) (end 54 98) (width 0.5) (layer "F.Cu") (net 20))
 (segment (start 54.75 81.21) (end 54.75 84.75) (width 0.5) (layer "F.Cu") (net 20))
 (segment (start 54.75 84.75) (end 54 85.5) (width 0.5) (layer "F.Cu") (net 20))
 (segment (start 53 79.46) (end 54.75 81.21) (width 0.5) (layer "F.Cu") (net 20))
 (segment (start 66 58.5) (end 66 52) (width 0.5) (layer "F.Cu") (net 19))
 (segment (start 53 82) (end 52 83) (width 0.5) (layer "F.Cu") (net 19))
 (segment (start 52 83) (end 52 98) (width 0.5) (layer "F.Cu") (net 19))
 (segment (start 55.2 66.9) (end 56.2 65.9) (width 0.5) (layer "B.Cu") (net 19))
 (segment (start 53 81.905) (end 54.3 80.605) (width 0.5) (layer "B.Cu") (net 19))
 (segment (start 55.2 70.48995) (end 55.2 66.9) (width 0.5) (layer "B.Cu") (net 19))
 (segment (start 66 60) (end 66 58.5) (width 0.5) (layer "B.Cu") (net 19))
 (segment (start 54.3 71.38995) (end 55.2 70.48995) (width 0.5) (layer "B.Cu") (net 19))
 (segment (start 60.1 65.9) (end 66 60) (width 0.5) (layer "B.Cu") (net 19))
 (segment (start 56.2 65.9) (end 60.1 65.9) (width 0.5) (layer "B.Cu") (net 19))
 (segment (start 54.3 80.605) (end 54.3 71.38995) (width 0.5) (layer "B.Cu") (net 19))
 (segment (start 58.352082 52.45) (end 59 53.097918) (width 0.3) (layer "F.Cu") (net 3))
 (segment (start 58 57.6) (end 59 56.6) (width 0.5) (layer "F.Cu") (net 3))
 (segment (start 59 53.097918) (end 59 53.1) (width 0.3) (layer "F.Cu") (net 3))
 (segment (start 53.53 55.5) (end 56.5 55.5) (width 0.3) (layer "F.Cu") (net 3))
 (segment (start 58 62.5) (end 58 57.6) (width 0.5) (layer "F.Cu") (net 3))
 (segment (start 58.3 55.9) (end 57.9 55.5) (width 0.3) (layer "F.Cu") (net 3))
 (segment (start 56.5 53) (end 53.53 53) (width 0.3) (layer "F.Cu") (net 3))
 (segment (start 57.05 52.45) (end 58.352082 52.45) (width 0.3) (layer "F.Cu") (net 3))
 (segment (start 56.5 55.5) (end 57.9 55.5) (width 0.3) (layer "F.Cu") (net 3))
 (segment (start 59 56.6) (end 58.3 55.9) (width 0.5) (layer "F.Cu") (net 3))
 (segment (start 56.5 53) (end 57.05 52.45) (width 0.3) (layer "F.Cu") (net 3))
 (segment (start 59 53.1) (end 59 56.6) (width 0.5) (layer "F.Cu") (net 3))
 (segment (start 53 71.84) (end 55.74 71.84) (width 0.5) (layer "F.Cu") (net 18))
 (segment (start 59.75 75.85) (end 59.75 97.75) (width 0.5) (layer "F.Cu") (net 18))
 (segment (start 55.74 71.84) (end 59.75 75.85) (width 0.5) (layer "F.Cu") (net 18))
 (segment (start 59.75 97.75) (end 60 98) (width 0.5) (layer "F.Cu") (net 18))
 (segment (start 62 61) (end 63.7 59.3) (width 0.5) (layer "B.Cu") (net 18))
 (segment (start 55.8 65.1) (end 59.65 65.1) (width 0.5) (layer "B.Cu") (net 18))
 (segment (start 54.4 70.3) (end 54.4 66.5) (width 0.5) (layer "B.Cu") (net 18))
 (segment (start 63.7 51.05) (end 65.75 49) (width 0.5) (layer "B.Cu") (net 18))
 (segment (start 63.7 59.3) (end 63.7 51.05) (width 0.5) (layer "B.Cu") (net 18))
 (segment (start 53 71.745) (end 53 71.7) (width 0.5) (layer "B.Cu") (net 18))
 (segment (start 53 71.7) (end 54.4 70.3) (width 0.5) (layer "B.Cu") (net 18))
 (segment (start 54.4 66.5) (end 55.8 65.1) (width 0.5) (layer "B.Cu") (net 18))
 (segment (start 59.65 65.1) (end 62 62.75) (width 0.5) (layer "B.Cu") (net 18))
 (segment (start 62 62.75) (end 62 61) (width 0.5) (layer "B.Cu") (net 18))
 (segment (start 59.9 78) (end 58.6 79.3) (width 0.5) (layer "B.Cu") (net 15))
 (segment (start 54 95.875) (end 54 98) (width 0.5) (layer "B.Cu") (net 15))
 (segment (start 59.9 71.86) (end 59.9 78) (width 0.5) (layer "B.Cu") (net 15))
 (segment (start 65 66.76) (end 59.9 71.86) (width 0.5) (layer "B.Cu") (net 15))
 (segment (start 58.6 79.3) (end 58.6 91.275) (width 0.5) (layer "B.Cu") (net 15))
 (segment (start 58.6 91.275) (end 54 95.875) (width 0.5) (layer "B.Cu") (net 15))
 (segment (start 65 64.925) (end 65 64.22) (width 0.5) (layer "B.Cu") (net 16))
 (segment (start 64.461522 65.46) (end 64.465 65.46) (width 0.5) (layer "B.Cu") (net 16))
 (segment (start 55.2 82.55) (end 55.2 74.725) (width 0.5) (layer "B.Cu") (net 16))
 (segment (start 63.7 66.225) (end 63.7 66.221522) (width 0.5) (layer "B.Cu") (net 16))
 (segment (start 63.7 66.221522) (end 64.461522 65.46) (width 0.5) (layer "B.Cu") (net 16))
 (segment (start 52 85.75) (end 55.2 82.55) (width 0.5) (layer "B.Cu") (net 16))
 (segment (start 55.2 74.725) (end 63.7 66.225) (width 0.5) (layer "B.Cu") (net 16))
 (segment (start 64.465 65.46) (end 65 64.925) (width 0.5) (layer "B.Cu") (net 16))
 (segment (start 52 98) (end 52 85.75) (width 0.5) (layer "B.Cu") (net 16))
 (segment (start 53.53 58.195) (end 53.585 58.25) (width 0.5) (layer "F.Cu") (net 2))
 (segment (start 56.66 78.04) (end 58 79.38) (width 0.5) (layer "F.Cu") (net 2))
 (segment (start 53.53 57) (end 53.53 58.195) (width 0.5) (layer "F.Cu") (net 2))
 (segment (start 56.445 58.25) (end 55.5075 59.1875) (width 0.5) (layer "F.Cu") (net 2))
 (segment (start 58.4 76.31) (end 56.67 78.04) (width 0.5) (layer "F.Cu") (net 2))
 (segment (start 56.5 58.195) (end 56.445 58.25) (width 0.5) (layer "F.Cu") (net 2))
 (segment (start 58 79.38) (end 58 98) (width 0.5) (layer "F.Cu") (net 2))
 (segment (start 61.5 52) (end 61.5 51.25) (width 0.5) (layer "F.Cu") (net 2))
 (segment (start 58.4 42.03) (end 58.4 42) (width 0.5) (layer "F.Cu") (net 2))
 (segment (start 56.445 46.015) (end 55.43 45) (width 0.5) (layer "F.Cu") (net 2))
 (segment (start 55.43 45) (end 58.4 42.03) (width 0.5) (layer "F.Cu") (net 2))
 (segment (start 56.67 78.04) (end 56.66 78.04) (width 0.5) (layer "F.Cu") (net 2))
 (segment (start 50.5 71.785) (end 50.5 63.75) (width 0.5) (layer "F.Cu") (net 2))
 (segment (start 53.585 46.845) (end 53.585 50.25) (width 0.5) (layer "F.Cu") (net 2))
 (segment (start 53 74.38) (end 55.26 76.64) (width 0.5) (layer "F.Cu") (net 2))
 (segment (start 50.5 63.75) (end 52.75 61.5) (width 0.5) (layer "F.Cu") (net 2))
 (segment (start 53 74.285) (end 53 74.38) (width 0.5) (layer "F.Cu") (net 2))
 (segment (start 56.5 51.5) (end 56.5 50.305) (width 0.5) (layer "F.Cu") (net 2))
 (segment (start 55.36 76.64) (end 55.26 76.64) (width 0.5) (layer "F.Cu") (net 2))
 (segment (start 56.5 50.305) (end 56.445 50.25) (width 0.5) (layer "F.Cu") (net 2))
 (segment (start 56.46 77.84) (end 56.66 78.04) (width 0.5) (layer "F.Cu") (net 2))
 (segment (start 56.4 75.6) (end 55.36 76.64) (width 0.5) (layer "F.Cu") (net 2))
 (segment (start 59 51.5) (end 57.695 51.5) (width 0.5) (layer "F.Cu") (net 2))
 (segment (start 52.36 42) (end 58.4 42) (width 0.5) (layer "F.Cu") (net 2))
 (segment (start 57.695 51.5) (end 56.445 50.25) (width 0.5) (layer "F.Cu") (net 2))
 (segment (start 53.53 51.5) (end 53.53 50.305) (width 0.5) (layer "F.Cu") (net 2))
 (segment (start 55.26 76.64) (end 56.46 77.84) (width 0.5) (layer "F.Cu") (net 2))
 (segment (start 61.25 58.25) (end 61.5 58.5) (width 0.5) (layer "F.Cu") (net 2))
 (segment (start 61.5 58.5) (end 61.5 52) (width 0.5) (layer "F.Cu") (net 2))
 (segment (start 58.4 42) (end 65.5 42) (width 0.5) (layer "F.Cu") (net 2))
 (segment (start 56.445 50.25) (end 56.445 46.015) (width 0.5) (layer "F.Cu") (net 2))
 (segment (start 53.53 57) (end 56.5 57) (width 0.5) (layer "F.Cu") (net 2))
 (segment (start 55.43 45) (end 53.585 46.845) (width 0.5) (layer "F.Cu") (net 2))
 (segment (start 53 74.285) (end 50.5 71.785) (width 0.5) (layer "F.Cu") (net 2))
 (segment (start 56.5 57) (end 56.5 58.195) (width 0.5) (layer "F.Cu") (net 2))
 (segment (start 56.5 51.5) (end 53.53 51.5) (width 0.5) (layer "F.Cu") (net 2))
 (segment (start 53.53 50.305) (end 53.585 50.25) (width 0.5) (layer "F.Cu") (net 2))
 (segment (start 54.5225 59.1875) (end 53.585 58.25) (width 0.5) (layer "F.Cu") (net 2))
 (segment (start 55.5075 59.1875) (end 54.5225 59.1875) (width 0.5) (layer "F.Cu") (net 2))
 (via (at 52.75 61.5) (size 1) (drill 0.5) (layers "F.Cu" "B.Cu") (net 2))
 (via (at 59 51.5) (size 1) (drill 0.5) (layers "F.Cu" "B.Cu") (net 2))
 (segment (start 56.445 58.25) (end 59 55.695) (width 0.5) (layer "B.Cu") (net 2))
 (segment (start 61.425 58.575) (end 61.5 58.5) (width 0.5) (layer "B.Cu") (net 2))
 (segment (start 54.584218 49.21) (end 53.585 50.209218) (width 0.5) (layer "B.Cu") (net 2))
 (segment (start 65.5 42) (end 65.5 46.25) (width 0.5) (layer "B.Cu") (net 2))
 (segment (start 60.925 51.425) (end 61.5 52) (width 0.5) (layer "B.Cu") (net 2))
 (segment (start 53.195 61.5) (end 56.445 58.25) (width 0.5) (layer "B.Cu") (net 2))
 (segment (start 56.445 50.209218) (end 55.445782 49.21) (width 0.5) (layer "B.Cu") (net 2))
 (segment (start 55.445782 49.21) (end 54.584218 49.21) (width 0.5) (layer "B.Cu") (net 2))
 (segment (start 61.25 58.25) (end 61.5 58.5) (width 0.5) (layer "B.Cu") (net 2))
 (segment (start 53.585 50.209218) (end 53.585 50.25) (width 0.5) (layer "B.Cu") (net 2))
 (segment (start 63.75 49) (end 63.75 49.75) (width 0.5) (layer "B.Cu") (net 2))
 (segment (start 59 55.695) (end 59 51.5) (width 0.5) (layer "B.Cu") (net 2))
 (segment (start 65.5 46.25) (end 63.75 48) (width 0.5) (layer "B.Cu") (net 2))
 (segment (start 56.445 58.25) (end 61.25 58.25) (width 0.5) (layer "B.Cu") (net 2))
 (segment (start 63.75 48) (end 63.75 49) (width 0.5) (layer "B.Cu") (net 2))
 (segment (start 52.75 61.5) (end 53.195 61.5) (width 0.5) (layer "B.Cu") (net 2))
 (segment (start 56.445 50.25) (end 56.445 50.209218) (width 0.5) (layer "B.Cu") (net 2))
 (segment (start 63.75 49.75) (end 61.5 52) (width 0.5) (layer "B.Cu") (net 2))
 (segment (start 56 98) (end 56 95.75) (width 0.5) (layer "B.Cu") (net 14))
 (segment (start 59.6 92.15) (end 59.6 79.6) (width 0.5) (layer "B.Cu") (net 14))
 (segment (start 60.8 73.5) (end 65 69.3) (width 0.5) (layer "B.Cu") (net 14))
 (segment (start 60.8 78.4) (end 60.8 73.5) (width 0.5) (layer "B.Cu") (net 14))
 (segment (start 56 95.75) (end 59.6 92.15) (width 0.5) (layer "B.Cu") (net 14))
 (segment (start 59.6 79.6) (end 60.8 78.4) (width 0.5) (layer "B.Cu") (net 14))
 (segment (start 52.6 55.15) (end 52.6 57.4) (width 0.3) (layer "F.Cu") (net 1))
 (segment (start 52.2975 59.2975) (end 56.4 63.4) (width 0.3) (layer "F.Cu") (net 1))
 (segment (start 52.2975 57.7025) (end 52.2975 59.2975) (width 0.3) (layer "F.Cu") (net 1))
 (segment (start 52.6 57.4) (end 52.2975 57.7025) (width 0.3) (layer "F.Cu") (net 1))
 (segment (start 52.75 55) (end 52.6 55.15) (width 0.3) (layer "F.Cu") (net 1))
 (segment (start 53.53 55) (end 52.75 55) (width 0.3) (layer "F.Cu") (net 1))
 (segment (start 56.4 63.4) (end 56.4 67.98) (width 0.3) (layer "F.Cu") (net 1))
 (segment (start 57.8 53.5) (end 58 53.3) (width 0.3) (layer "F.Cu") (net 7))
 (segment (start 56.5 53.5) (end 57.8 53.5) (width 0.3) (layer "F.Cu") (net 7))
 (via (at 58 53.3) (size 1) (drill 0.5) (layers "F.Cu" "B.Cu") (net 7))
 (segment (start 60.6 46.4) (end 63.4 46.4) (width 0.3) (layer "B.Cu") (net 7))
 (segment (start 67.523 59.567) (end 58.4 68.69) (width 0.3) (layer "B.Cu") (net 7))
 (segment (start 64.662045 39.977) (end 66.337955 39.977) (width 0.3) (layer "B.Cu") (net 7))
 (segment (start 67.523 41.162045) (end 67.523 59.567) (width 0.3) (layer "B.Cu") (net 7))
 (segment (start 63.4 46.4) (end 63.9 45.9) (width 0.3) (layer "B.Cu") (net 7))
 (segment (start 58 49) (end 60.6 46.4) (width 0.3) (layer "B.Cu") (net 7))
 (segment (start 63.477 41.162045) (end 64.662045 39.977) (width 0.3) (layer "B.Cu") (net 7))
 (segment (start 58 53.3) (end 58 49) (width 0.3) (layer "B.Cu") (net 7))
 (segment (start 66.337955 39.977) (end 67.523 41.162045) (width 0.3) (layer "B.Cu") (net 7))
 (segment (start 63.9 43.260955) (end 63.477 42.837955) (width 0.3) (layer "B.Cu") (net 7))
 (segment (start 63.9 45.9) (end 63.9 43.260955) (width 0.3) (layer "B.Cu") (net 7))
 (segment (start 63.477 42.837955) (end 63.477 41.162045) (width 0.3) (layer "B.Cu") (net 7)))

